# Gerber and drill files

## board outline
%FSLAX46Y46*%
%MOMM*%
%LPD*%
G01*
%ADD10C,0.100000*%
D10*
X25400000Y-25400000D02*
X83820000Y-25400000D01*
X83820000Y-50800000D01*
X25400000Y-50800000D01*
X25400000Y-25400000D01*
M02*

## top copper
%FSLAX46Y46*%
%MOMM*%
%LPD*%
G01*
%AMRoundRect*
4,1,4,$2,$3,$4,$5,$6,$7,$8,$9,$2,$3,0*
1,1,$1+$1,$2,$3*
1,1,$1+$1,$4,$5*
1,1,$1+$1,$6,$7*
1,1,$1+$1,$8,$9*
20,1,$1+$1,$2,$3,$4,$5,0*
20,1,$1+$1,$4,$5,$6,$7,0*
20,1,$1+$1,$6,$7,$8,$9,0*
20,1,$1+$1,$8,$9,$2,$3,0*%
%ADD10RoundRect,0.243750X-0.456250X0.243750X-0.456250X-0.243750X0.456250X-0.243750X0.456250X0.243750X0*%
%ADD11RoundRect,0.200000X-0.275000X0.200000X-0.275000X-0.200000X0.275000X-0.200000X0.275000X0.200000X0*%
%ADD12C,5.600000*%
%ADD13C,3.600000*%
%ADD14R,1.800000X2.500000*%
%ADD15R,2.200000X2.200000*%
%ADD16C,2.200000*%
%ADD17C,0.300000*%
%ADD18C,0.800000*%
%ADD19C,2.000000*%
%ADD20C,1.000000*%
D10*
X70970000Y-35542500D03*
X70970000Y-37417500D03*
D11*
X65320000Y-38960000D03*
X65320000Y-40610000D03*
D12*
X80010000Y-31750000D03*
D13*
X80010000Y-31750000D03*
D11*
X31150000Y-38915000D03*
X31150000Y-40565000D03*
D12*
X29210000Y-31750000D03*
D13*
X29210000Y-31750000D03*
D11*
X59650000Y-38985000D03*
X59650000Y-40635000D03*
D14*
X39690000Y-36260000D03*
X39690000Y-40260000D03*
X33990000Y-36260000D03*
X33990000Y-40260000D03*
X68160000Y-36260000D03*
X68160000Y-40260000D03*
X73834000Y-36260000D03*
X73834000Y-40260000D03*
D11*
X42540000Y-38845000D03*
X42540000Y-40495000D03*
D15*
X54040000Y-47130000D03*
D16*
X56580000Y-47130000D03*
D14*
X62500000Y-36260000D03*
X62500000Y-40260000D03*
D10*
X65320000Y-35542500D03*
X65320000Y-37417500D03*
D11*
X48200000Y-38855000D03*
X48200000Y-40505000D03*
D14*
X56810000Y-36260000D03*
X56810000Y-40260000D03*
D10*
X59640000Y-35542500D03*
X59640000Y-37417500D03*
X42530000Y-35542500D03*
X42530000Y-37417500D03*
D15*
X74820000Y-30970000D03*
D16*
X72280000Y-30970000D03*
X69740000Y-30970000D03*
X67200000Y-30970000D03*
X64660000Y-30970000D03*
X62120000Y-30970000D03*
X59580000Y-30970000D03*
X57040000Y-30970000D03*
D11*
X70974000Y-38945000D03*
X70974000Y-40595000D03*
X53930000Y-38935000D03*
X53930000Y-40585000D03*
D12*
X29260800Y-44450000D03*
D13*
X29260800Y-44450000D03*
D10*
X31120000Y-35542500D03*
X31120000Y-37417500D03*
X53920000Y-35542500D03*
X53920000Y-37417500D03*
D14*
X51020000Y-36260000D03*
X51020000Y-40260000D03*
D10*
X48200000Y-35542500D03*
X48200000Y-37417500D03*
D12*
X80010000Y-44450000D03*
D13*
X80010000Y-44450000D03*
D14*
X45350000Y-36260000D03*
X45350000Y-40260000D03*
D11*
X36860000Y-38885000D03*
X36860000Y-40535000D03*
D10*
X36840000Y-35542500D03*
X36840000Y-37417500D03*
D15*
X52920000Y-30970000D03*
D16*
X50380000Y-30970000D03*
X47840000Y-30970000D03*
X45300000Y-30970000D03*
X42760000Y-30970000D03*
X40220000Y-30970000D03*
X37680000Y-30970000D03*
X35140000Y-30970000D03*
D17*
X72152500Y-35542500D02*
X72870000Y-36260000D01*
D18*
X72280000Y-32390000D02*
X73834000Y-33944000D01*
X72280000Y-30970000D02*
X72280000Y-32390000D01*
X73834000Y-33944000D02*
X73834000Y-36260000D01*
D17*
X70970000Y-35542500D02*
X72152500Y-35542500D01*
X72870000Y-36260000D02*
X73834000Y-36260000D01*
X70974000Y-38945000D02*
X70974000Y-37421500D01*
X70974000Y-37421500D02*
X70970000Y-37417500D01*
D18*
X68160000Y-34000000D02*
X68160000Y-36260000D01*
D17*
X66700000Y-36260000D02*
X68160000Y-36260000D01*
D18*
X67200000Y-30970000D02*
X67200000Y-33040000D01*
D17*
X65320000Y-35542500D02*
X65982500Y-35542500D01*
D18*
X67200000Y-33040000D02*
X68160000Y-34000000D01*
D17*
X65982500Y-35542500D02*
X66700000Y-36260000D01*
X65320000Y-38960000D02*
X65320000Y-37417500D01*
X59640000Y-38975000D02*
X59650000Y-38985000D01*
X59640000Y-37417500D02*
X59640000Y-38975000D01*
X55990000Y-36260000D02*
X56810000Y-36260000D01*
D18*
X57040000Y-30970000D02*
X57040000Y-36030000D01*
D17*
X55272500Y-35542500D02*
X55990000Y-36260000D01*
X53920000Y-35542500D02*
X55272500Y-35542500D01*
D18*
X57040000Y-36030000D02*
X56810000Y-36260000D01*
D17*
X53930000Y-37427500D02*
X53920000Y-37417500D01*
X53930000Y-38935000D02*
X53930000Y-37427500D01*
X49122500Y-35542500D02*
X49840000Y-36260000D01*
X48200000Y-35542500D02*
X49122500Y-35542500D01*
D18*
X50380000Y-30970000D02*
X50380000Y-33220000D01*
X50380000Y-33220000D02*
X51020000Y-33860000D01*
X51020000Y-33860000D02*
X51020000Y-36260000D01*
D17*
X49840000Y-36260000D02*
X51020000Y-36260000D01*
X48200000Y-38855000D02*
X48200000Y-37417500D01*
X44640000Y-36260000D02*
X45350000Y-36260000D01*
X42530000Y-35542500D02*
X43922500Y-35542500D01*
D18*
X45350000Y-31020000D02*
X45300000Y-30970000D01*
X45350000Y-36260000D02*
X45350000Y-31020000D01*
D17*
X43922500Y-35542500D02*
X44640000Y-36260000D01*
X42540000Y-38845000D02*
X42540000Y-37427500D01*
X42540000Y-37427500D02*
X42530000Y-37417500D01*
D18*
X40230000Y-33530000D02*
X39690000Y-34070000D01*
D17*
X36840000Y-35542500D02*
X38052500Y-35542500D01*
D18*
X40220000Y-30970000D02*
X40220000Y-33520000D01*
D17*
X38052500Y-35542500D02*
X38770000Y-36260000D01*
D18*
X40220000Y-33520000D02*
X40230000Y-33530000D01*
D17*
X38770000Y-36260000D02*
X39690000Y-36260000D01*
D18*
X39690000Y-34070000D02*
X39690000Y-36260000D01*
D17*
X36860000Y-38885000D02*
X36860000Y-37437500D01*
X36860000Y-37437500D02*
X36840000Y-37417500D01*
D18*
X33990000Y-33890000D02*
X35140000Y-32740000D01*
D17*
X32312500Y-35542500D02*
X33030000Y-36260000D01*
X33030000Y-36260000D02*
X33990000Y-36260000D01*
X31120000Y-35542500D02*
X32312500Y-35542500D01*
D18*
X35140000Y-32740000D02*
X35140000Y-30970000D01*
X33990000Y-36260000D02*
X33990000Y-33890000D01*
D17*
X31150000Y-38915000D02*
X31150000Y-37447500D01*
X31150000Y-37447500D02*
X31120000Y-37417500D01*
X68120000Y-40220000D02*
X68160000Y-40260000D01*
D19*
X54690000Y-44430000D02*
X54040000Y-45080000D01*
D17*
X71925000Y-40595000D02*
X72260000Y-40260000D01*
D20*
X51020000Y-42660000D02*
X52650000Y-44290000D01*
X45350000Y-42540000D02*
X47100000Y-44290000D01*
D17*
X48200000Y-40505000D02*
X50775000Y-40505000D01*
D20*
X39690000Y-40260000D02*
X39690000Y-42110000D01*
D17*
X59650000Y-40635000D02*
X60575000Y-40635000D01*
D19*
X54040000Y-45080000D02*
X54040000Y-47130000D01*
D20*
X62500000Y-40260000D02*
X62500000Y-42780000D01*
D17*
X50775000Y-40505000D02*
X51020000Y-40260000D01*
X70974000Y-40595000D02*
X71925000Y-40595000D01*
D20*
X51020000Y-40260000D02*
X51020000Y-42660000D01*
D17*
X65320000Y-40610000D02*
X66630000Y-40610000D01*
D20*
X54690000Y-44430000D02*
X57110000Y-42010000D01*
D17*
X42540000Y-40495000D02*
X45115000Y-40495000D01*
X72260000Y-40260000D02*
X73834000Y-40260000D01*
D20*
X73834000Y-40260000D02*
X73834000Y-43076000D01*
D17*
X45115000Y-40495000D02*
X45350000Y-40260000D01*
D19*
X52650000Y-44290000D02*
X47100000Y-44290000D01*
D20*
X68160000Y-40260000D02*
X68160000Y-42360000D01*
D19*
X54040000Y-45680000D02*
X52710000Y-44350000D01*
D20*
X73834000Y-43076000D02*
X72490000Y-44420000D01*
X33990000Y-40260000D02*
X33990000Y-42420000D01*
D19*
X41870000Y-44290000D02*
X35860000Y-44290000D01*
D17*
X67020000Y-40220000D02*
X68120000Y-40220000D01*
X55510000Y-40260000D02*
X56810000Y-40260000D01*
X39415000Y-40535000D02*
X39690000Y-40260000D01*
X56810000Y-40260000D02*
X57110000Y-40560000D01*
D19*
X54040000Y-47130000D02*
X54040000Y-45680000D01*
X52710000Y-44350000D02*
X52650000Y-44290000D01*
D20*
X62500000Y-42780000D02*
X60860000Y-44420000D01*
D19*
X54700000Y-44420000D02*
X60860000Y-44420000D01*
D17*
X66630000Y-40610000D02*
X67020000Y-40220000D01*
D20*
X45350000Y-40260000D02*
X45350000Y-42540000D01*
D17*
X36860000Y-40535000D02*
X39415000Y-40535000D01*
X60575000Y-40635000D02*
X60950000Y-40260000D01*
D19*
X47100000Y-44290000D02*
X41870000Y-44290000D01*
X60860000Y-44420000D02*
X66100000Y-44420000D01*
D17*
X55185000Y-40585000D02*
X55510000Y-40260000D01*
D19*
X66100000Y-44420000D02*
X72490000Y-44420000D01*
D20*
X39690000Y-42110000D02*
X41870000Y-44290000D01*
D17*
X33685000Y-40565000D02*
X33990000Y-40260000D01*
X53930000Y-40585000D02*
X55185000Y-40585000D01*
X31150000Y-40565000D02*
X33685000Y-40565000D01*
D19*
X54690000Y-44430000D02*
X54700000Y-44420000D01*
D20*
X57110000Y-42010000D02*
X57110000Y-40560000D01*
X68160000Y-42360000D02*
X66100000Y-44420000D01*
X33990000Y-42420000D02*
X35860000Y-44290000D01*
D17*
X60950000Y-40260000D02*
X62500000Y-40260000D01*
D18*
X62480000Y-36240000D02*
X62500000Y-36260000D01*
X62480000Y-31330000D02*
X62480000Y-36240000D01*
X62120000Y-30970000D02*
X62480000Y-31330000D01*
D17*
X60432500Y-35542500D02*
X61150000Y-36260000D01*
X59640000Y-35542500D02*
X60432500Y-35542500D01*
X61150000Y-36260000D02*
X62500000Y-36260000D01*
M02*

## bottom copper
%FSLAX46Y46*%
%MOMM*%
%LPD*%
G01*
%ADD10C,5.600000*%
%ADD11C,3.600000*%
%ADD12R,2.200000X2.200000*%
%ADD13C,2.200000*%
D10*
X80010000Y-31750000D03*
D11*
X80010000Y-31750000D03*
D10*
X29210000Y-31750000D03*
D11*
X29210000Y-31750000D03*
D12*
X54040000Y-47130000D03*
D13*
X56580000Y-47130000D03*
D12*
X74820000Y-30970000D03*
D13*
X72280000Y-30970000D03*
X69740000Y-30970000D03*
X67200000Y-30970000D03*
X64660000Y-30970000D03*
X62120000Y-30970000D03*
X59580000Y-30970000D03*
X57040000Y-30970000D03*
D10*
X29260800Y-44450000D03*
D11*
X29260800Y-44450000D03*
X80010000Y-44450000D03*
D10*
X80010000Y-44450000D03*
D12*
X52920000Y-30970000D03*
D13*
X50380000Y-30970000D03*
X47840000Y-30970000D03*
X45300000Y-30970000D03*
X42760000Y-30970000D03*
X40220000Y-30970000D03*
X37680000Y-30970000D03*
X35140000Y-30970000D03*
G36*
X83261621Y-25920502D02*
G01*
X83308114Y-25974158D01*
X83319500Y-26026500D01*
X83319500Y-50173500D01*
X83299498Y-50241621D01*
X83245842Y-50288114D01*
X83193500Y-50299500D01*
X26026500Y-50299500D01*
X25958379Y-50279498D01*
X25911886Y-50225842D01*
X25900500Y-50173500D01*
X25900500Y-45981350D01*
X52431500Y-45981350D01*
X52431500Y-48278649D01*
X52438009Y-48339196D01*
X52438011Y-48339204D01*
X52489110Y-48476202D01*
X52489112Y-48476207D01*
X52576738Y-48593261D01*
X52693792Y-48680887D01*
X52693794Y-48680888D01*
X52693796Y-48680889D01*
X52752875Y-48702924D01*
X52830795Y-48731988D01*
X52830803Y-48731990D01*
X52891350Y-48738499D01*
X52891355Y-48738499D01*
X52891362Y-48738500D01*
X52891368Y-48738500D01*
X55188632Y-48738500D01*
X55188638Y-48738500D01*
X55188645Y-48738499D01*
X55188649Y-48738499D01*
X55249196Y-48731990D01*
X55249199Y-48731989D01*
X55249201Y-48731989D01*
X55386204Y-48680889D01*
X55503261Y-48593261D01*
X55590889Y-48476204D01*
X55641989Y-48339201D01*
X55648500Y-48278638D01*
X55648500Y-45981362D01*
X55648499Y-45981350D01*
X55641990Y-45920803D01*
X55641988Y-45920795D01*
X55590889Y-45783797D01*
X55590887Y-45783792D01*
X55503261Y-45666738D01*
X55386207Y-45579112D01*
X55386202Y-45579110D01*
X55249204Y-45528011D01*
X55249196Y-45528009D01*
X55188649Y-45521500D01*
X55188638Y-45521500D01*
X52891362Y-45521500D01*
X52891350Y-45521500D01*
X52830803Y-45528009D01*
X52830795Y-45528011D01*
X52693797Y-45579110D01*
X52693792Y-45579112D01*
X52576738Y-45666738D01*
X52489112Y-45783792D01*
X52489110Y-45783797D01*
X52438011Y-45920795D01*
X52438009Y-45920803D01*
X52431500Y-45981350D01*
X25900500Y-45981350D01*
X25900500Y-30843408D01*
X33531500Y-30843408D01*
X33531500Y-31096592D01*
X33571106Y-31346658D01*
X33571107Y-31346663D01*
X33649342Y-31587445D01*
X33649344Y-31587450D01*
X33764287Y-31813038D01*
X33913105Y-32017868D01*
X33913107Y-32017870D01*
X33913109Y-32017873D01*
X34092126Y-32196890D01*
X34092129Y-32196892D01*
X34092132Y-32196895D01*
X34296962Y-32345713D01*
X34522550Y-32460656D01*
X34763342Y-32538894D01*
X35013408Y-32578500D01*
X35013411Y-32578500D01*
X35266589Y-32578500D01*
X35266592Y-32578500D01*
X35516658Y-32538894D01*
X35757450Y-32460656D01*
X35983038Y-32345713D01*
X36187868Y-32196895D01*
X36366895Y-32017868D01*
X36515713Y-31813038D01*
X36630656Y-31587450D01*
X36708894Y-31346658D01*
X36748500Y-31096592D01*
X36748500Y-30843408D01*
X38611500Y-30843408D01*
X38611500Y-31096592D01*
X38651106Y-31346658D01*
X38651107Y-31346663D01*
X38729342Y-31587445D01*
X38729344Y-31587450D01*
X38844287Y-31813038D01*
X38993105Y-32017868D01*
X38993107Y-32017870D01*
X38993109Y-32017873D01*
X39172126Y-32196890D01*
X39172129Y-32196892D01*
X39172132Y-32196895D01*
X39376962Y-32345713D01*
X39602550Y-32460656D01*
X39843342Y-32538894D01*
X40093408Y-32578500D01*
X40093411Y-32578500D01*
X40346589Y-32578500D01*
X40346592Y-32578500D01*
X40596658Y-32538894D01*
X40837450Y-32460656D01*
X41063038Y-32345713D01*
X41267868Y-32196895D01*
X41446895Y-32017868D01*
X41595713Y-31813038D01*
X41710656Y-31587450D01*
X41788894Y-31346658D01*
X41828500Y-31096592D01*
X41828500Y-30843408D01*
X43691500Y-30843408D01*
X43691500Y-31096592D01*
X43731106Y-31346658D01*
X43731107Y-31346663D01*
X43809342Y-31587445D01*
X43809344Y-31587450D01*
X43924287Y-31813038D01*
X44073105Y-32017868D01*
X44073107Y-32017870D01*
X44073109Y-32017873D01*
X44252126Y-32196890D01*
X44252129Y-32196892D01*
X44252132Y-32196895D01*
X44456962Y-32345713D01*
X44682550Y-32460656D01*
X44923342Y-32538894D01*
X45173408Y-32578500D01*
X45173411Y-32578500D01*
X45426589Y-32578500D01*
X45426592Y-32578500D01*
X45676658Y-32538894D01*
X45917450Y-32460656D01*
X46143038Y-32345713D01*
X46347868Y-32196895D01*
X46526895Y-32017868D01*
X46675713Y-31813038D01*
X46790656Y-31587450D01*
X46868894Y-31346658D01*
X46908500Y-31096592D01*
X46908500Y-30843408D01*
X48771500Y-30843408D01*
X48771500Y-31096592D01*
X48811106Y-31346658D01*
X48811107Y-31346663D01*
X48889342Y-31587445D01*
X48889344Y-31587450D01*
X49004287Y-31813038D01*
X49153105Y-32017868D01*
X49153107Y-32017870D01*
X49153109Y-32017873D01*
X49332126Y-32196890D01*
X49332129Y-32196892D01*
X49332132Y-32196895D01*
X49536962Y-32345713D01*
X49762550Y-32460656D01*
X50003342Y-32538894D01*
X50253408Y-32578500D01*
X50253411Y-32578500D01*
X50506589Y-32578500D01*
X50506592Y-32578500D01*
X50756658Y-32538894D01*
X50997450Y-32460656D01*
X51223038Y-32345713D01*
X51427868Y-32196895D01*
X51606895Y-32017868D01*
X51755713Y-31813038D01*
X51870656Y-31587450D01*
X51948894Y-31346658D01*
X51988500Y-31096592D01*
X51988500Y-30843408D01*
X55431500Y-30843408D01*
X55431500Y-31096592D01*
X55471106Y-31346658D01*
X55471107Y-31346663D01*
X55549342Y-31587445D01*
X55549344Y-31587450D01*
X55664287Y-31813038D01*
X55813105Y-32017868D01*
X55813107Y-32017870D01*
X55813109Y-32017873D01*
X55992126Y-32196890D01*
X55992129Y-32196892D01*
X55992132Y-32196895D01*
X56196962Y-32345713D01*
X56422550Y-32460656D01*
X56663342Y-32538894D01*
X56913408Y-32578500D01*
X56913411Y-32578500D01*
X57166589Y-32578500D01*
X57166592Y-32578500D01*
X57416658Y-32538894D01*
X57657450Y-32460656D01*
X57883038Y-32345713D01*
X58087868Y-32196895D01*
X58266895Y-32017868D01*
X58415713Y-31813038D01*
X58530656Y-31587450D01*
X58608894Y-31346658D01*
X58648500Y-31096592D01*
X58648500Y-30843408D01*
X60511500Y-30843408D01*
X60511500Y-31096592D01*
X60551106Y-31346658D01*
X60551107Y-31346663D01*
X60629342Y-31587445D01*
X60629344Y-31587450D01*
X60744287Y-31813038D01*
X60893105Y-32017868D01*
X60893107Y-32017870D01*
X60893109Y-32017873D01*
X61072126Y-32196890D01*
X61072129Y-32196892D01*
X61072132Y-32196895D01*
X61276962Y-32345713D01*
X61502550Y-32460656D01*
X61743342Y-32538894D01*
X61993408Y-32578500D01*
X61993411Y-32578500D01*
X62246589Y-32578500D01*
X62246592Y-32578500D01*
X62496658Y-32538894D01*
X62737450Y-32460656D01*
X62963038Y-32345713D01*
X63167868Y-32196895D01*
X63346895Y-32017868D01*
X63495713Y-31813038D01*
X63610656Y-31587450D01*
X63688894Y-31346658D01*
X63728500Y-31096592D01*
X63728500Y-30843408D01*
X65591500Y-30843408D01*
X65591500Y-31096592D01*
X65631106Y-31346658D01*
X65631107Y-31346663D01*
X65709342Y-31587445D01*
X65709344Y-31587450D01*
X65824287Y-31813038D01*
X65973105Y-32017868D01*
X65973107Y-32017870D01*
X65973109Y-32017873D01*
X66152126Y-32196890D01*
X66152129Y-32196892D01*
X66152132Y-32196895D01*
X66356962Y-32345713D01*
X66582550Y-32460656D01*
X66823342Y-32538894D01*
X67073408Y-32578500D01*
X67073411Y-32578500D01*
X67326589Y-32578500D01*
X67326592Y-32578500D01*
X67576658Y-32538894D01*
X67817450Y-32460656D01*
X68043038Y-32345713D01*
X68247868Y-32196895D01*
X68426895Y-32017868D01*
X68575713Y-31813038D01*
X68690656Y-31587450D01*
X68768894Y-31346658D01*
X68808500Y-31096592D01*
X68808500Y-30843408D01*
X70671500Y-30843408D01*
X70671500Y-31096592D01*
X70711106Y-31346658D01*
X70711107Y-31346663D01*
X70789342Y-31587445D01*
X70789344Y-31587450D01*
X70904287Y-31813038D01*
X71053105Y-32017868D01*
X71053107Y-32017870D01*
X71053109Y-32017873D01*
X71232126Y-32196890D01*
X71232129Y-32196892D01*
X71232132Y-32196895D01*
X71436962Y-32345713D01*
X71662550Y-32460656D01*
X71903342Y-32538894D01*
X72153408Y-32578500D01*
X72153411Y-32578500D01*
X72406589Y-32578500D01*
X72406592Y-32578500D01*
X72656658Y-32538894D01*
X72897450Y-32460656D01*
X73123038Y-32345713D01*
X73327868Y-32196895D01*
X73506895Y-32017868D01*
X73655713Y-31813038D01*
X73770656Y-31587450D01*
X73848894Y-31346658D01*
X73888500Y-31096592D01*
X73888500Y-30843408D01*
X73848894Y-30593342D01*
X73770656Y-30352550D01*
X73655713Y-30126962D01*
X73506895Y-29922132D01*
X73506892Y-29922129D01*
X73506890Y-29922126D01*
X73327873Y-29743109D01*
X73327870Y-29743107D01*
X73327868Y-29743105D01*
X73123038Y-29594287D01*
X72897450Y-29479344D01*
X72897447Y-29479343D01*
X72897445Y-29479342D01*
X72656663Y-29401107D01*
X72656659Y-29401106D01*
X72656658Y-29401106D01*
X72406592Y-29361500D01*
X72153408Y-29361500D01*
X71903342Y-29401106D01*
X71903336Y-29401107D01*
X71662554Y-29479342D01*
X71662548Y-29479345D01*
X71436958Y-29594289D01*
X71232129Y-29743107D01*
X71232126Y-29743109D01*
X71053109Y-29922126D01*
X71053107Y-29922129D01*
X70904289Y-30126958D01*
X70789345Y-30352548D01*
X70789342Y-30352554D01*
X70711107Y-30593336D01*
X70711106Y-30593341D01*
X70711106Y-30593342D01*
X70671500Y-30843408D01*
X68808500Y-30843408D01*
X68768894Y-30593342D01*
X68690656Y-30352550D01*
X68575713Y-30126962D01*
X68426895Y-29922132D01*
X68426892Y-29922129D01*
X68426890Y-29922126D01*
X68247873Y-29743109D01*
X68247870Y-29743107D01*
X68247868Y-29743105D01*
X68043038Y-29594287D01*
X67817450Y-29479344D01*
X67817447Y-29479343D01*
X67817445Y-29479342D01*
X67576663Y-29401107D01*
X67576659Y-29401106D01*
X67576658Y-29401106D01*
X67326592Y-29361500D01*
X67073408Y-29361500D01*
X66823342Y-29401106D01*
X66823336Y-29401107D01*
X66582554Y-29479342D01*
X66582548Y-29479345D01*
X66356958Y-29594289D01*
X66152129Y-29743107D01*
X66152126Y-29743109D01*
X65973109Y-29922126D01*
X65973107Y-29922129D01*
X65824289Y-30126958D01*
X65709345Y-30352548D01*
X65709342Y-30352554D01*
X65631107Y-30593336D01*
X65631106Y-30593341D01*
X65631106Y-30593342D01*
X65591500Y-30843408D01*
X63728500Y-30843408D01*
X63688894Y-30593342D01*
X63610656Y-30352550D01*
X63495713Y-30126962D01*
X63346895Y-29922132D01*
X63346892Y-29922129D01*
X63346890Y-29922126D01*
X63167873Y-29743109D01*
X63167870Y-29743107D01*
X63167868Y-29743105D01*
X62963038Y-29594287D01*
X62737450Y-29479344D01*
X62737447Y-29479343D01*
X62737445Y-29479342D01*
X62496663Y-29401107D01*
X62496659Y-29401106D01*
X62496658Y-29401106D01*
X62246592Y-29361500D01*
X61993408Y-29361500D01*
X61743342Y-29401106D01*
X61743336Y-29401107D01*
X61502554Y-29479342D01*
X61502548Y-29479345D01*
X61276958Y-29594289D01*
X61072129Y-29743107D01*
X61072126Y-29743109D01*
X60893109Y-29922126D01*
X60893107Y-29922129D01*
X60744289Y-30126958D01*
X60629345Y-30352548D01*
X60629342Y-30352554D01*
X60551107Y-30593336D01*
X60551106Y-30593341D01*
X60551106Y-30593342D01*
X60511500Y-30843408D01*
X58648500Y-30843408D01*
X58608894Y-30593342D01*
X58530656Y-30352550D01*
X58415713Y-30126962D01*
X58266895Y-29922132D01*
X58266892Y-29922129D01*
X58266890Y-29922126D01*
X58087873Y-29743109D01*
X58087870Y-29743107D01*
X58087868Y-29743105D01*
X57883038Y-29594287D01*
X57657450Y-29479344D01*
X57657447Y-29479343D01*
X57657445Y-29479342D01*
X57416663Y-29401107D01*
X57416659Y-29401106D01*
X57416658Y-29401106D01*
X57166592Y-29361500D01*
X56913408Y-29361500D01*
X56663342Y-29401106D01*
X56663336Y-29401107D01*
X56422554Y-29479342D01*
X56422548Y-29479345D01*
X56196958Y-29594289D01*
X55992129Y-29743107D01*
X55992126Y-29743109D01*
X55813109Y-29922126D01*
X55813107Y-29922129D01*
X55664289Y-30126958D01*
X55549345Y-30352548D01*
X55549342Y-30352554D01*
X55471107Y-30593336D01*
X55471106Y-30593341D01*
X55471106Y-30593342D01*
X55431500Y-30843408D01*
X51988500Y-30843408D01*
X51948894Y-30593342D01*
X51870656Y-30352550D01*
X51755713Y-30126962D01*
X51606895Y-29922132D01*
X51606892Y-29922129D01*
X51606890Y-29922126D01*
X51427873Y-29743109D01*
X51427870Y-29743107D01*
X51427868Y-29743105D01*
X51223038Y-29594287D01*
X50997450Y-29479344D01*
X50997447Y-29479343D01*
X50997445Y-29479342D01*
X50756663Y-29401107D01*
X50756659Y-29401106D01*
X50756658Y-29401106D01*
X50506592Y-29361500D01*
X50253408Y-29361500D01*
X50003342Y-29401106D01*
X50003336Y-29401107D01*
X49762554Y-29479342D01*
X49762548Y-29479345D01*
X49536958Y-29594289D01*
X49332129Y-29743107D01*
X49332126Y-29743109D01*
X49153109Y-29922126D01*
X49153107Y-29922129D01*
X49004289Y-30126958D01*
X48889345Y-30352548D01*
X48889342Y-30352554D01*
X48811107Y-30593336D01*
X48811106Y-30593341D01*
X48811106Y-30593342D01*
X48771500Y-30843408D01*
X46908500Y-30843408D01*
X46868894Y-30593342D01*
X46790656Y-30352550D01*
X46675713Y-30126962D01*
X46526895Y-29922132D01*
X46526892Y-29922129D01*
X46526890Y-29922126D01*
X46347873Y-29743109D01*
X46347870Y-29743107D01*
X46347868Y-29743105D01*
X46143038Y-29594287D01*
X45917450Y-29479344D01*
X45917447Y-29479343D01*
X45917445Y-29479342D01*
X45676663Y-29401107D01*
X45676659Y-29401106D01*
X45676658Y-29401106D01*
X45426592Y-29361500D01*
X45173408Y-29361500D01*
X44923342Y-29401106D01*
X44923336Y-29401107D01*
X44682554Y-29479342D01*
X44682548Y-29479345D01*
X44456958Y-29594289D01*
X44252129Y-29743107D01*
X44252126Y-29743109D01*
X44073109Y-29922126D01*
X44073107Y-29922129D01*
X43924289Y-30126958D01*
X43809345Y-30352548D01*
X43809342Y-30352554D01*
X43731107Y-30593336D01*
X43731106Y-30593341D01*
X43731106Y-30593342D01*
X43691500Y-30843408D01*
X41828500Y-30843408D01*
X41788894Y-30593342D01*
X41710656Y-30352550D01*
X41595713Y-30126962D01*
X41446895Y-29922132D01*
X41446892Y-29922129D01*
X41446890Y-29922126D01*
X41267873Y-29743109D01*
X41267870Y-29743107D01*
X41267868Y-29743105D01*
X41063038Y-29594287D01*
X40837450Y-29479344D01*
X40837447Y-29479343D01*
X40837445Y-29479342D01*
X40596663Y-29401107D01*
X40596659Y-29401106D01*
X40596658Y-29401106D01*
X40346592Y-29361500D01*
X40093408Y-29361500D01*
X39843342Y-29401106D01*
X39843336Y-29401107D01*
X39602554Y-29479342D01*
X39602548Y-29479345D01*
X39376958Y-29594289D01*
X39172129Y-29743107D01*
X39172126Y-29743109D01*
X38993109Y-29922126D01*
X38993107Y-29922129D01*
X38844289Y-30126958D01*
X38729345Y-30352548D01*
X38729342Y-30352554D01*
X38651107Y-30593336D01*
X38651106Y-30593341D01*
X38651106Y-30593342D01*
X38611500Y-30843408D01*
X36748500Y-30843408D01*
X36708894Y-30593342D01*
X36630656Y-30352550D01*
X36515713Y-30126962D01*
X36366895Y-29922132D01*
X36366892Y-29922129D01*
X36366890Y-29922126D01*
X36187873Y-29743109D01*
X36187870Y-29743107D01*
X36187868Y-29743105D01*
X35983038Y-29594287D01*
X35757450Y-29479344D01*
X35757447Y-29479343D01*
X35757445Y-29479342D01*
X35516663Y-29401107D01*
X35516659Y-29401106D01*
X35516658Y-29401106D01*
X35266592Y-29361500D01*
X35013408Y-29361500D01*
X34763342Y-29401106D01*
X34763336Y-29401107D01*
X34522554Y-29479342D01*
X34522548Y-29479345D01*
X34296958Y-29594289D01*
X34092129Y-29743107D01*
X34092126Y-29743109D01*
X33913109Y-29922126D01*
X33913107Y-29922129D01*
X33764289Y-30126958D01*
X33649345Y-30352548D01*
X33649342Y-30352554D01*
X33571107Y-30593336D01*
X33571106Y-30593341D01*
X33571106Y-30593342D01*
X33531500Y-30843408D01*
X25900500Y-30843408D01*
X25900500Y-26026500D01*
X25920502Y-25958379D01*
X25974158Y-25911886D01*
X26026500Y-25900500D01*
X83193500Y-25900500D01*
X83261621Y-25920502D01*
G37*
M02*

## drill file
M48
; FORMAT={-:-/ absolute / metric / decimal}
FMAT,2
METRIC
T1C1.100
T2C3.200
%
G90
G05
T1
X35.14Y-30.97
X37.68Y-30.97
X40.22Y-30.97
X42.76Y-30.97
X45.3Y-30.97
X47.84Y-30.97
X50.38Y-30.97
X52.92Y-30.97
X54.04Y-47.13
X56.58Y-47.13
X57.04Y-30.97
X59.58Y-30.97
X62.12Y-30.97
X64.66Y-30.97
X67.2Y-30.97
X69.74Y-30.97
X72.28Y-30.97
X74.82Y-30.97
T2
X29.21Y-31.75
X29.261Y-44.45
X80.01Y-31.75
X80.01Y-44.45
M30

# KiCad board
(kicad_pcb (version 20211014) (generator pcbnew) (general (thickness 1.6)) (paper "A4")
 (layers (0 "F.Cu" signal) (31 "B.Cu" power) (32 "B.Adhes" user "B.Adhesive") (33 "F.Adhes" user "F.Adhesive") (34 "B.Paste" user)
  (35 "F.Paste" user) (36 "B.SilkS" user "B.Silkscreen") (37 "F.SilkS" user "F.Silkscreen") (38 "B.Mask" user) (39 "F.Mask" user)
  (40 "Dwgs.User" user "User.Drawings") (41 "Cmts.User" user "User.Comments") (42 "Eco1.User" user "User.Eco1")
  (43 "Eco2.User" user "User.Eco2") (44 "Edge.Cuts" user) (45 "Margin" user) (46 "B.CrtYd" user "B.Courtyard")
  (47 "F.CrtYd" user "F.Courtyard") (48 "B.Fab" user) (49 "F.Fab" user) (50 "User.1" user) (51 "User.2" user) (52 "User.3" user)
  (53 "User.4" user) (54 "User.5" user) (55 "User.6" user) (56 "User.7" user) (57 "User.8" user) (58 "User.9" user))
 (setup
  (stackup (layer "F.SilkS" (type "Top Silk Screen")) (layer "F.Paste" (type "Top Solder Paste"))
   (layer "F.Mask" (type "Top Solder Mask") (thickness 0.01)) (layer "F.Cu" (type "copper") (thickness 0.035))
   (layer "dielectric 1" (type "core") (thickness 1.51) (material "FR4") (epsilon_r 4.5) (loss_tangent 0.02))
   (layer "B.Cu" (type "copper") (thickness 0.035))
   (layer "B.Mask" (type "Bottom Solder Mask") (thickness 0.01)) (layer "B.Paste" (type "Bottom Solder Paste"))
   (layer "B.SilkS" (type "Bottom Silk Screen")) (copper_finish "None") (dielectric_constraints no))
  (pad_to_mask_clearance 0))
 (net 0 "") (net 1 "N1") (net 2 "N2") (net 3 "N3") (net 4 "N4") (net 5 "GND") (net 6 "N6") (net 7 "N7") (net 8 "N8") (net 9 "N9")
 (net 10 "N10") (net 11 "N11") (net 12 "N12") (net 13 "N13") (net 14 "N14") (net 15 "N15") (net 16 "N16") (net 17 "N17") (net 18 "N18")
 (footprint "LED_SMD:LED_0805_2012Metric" (layer "F.Cu") (at 70.97 36.48 -90)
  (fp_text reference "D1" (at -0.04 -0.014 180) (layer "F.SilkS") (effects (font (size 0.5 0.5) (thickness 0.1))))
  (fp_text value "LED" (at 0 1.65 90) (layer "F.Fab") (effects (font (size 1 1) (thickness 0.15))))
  (pad "1" smd roundrect (at -0.9375 0 270) (size 0.975 1.4) (layers "F.Cu" "F.Paste" "F.Mask") (roundrect_rratio 0.25) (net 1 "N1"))
  (pad "2" smd roundrect (at 0.9375 0 270) (size 0.975 1.4) (layers "F.Cu" "F.Paste" "F.Mask") (roundrect_rratio 0.25) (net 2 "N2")))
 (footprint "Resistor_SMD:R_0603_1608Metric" (layer "F.Cu") (at 65.32 39.785 -90)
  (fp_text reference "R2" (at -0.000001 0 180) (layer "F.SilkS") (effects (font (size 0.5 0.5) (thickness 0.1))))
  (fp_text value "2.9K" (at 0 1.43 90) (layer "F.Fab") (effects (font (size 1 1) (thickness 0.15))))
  (pad "1" smd roundrect (at -0.825 0 270) (size 0.8 0.95) (layers "F.Cu" "F.Paste" "F.Mask") (roundrect_rratio 0.25) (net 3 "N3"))
  (pad "2" smd roundrect (at 0.825 0 270) (size 0.8 0.95) (layers "F.Cu" "F.Paste" "F.Mask") (roundrect_rratio 0.25) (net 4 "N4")))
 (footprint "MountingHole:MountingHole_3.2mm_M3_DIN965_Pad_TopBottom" (layer "F.Cu") (at 80.01 31.75)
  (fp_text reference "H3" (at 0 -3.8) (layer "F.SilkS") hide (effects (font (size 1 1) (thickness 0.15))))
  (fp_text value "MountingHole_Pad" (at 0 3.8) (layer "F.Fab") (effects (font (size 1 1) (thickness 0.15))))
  (pad "1" connect circle (at 0 0) (size 5.6 5.6) (layers "B.Cu" "B.Mask") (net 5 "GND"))
  (pad "1" connect circle (at 0 0) (size 5.6 5.6) (layers "F.Cu" "F.Mask") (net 5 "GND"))
  (pad "1" thru_hole circle (at 0 0) (size 3.6 3.6) (drill 3.2) (layers *.Cu *.Mask) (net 5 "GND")))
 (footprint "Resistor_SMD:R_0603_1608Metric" (layer "F.Cu") (at 31.15 39.74 -90)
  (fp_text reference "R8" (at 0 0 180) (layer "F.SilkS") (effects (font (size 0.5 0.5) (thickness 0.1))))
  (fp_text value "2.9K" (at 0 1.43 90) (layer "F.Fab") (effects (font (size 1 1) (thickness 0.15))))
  (pad "1" smd roundrect (at -0.825 0 270) (size 0.8 0.95) (layers "F.Cu" "F.Paste" "F.Mask") (roundrect_rratio 0.25) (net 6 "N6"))
  (pad "2" smd roundrect (at 0.825 0 270) (size 0.8 0.95) (layers "F.Cu" "F.Paste" "F.Mask") (roundrect_rratio 0.25) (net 4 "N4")))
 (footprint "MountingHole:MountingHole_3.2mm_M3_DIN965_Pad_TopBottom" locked (layer "F.Cu") (at 29.21 31.75)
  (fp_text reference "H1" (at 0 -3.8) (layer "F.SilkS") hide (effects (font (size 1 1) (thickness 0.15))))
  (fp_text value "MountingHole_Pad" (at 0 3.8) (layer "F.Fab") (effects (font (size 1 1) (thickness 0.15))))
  (pad "1" connect circle locked (at 0 0) (size 5.6 5.6) (layers "F.Cu" "F.Mask") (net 5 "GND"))
  (pad "1" connect circle locked (at 0 0) (size 5.6 5.6) (layers "B.Cu" "B.Mask") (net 5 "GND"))
  (pad "1" thru_hole circle locked (at 0 0) (size 3.6 3.6) (drill 3.2) (layers *.Cu *.Mask) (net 5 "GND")))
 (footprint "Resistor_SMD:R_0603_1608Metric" (layer "F.Cu") (at 59.65 39.81 -90)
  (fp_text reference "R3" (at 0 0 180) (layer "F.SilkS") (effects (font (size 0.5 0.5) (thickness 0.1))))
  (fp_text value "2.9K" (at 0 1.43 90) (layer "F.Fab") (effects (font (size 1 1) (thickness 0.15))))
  (pad "1" smd roundrect (at -0.825 0 270) (size 0.8 0.95) (layers "F.Cu" "F.Paste" "F.Mask") (roundrect_rratio 0.25) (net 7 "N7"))
  (pad "2" smd roundrect (at 0.825 0 270) (size 0.8 0.95) (layers "F.Cu" "F.Paste" "F.Mask") (roundrect_rratio 0.25) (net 4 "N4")))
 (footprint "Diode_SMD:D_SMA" (layer "F.Cu") (at 39.69 38.26 -90)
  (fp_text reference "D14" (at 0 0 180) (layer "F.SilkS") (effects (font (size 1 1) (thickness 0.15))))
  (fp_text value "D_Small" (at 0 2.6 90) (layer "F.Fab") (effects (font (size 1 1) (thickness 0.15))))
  (pad "1" smd rect (at -2 0 270) (size 2.5 1.8) (layers "F.Cu" "F.Paste" "F.Mask") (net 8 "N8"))
  (pad "2" smd rect (at 2 0 270) (size 2.5 1.8) (layers "F.Cu" "F.Paste" "F.Mask") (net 4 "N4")))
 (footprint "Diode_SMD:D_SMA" (layer "F.Cu") (at 33.99 38.26 -90)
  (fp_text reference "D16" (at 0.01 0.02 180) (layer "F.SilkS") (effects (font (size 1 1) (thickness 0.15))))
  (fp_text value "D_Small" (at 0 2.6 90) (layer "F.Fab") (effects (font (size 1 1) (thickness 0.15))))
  (pad "1" smd rect (at -2 0 270) (size 2.5 1.8) (layers "F.Cu" "F.Paste" "F.Mask") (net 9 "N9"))
  (pad "2" smd rect (at 2 0 270) (size 2.5 1.8) (layers "F.Cu" "F.Paste" "F.Mask") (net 4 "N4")))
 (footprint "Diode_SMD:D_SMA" (layer "F.Cu") (at 68.16 38.26 -90)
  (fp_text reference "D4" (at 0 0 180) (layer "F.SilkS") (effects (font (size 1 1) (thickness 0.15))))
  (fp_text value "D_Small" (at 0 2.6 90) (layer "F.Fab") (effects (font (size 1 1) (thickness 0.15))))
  (pad "1" smd rect (at -2 0 270) (size 2.5 1.8) (layers "F.Cu" "F.Paste" "F.Mask") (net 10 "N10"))
  (pad "2" smd rect (at 2 0 270) (size 2.5 1.8) (layers "F.Cu" "F.Paste" "F.Mask") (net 4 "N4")))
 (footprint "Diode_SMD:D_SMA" (layer "F.Cu") (at 73.834 38.26 -90)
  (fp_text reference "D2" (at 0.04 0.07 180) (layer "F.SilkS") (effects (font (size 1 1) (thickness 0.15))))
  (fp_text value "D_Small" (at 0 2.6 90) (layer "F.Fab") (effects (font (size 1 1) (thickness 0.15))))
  (pad "1" smd rect (at -2 0 270) (size 2.5 1.8) (layers "F.Cu" "F.Paste" "F.Mask") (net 1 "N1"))
  (pad "2" smd rect (at 2 0 270) (size 2.5 1.8) (layers "F.Cu" "F.Paste" "F.Mask") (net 4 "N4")))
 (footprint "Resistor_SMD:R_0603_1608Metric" (layer "F.Cu") (at 42.54 39.67 -90)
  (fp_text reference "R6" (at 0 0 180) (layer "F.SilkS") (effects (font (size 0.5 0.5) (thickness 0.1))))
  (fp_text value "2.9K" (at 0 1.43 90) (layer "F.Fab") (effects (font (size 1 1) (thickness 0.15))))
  (pad "1" smd roundrect (at -0.825 0 270) (size 0.8 0.95) (layers "F.Cu" "F.Paste" "F.Mask") (roundrect_rratio 0.25) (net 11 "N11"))
  (pad "2" smd roundrect (at 0.825 0 270) (size 0.8 0.95) (layers "F.Cu" "F.Paste" "F.Mask") (roundrect_rratio 0.25) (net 4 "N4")))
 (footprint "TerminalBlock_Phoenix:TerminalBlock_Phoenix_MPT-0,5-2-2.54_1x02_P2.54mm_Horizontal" (layer "F.Cu") (at 54.04 47.13)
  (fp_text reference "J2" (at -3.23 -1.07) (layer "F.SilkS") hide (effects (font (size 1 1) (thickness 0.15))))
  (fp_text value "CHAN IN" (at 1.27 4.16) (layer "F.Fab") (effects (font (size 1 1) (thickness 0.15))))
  (pad "1" thru_hole rect (at 0 0) (size 2.2 2.2) (drill 1.1) (layers *.Cu *.Mask) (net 4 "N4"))
  (pad "2" thru_hole circle (at 2.54 0) (size 2.2 2.2) (drill 1.1) (layers *.Cu *.Mask) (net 5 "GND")))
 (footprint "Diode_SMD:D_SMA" (layer "F.Cu") (at 62.5 38.26 -90)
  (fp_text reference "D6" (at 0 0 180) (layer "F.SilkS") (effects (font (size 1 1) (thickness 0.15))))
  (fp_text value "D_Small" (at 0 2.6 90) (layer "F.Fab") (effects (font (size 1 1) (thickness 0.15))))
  (pad "1" smd rect (at -2 0 270) (size 2.5 1.8) (layers "F.Cu" "F.Paste" "F.Mask") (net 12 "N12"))
  (pad "2" smd rect (at 2 0 270) (size 2.5 1.8) (layers "F.Cu" "F.Paste" "F.Mask") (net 4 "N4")))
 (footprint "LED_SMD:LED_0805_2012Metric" (layer "F.Cu") (at 65.32 36.48 -90)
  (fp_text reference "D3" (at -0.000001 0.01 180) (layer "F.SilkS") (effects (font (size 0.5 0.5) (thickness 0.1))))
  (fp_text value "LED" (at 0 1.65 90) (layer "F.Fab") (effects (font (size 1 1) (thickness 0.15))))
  (pad "1" smd roundrect (at -0.9375 0 270) (size 0.975 1.4) (layers "F.Cu" "F.Paste" "F.Mask") (roundrect_rratio 0.25) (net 10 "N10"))
  (pad "2" smd roundrect (at 0.9375 0 270) (size 0.975 1.4) (layers "F.Cu" "F.Paste" "F.Mask") (roundrect_rratio 0.25) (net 3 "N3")))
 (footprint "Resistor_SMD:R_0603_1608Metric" (layer "F.Cu") (at 48.2 39.68 -90)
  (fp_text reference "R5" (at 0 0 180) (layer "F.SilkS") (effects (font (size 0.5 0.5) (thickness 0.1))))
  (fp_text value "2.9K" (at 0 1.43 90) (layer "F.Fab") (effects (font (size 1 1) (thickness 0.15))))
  (pad "1" smd roundrect (at -0.825 0 270) (size 0.8 0.95) (layers "F.Cu" "F.Paste" "F.Mask") (roundrect_rratio 0.25) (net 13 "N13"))
  (pad "2" smd roundrect (at 0.825 0 270) (size 0.8 0.95) (layers "F.Cu" "F.Paste" "F.Mask") (roundrect_rratio 0.25) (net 4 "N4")))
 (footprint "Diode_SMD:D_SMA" (layer "F.Cu") (at 56.81 38.26 -90)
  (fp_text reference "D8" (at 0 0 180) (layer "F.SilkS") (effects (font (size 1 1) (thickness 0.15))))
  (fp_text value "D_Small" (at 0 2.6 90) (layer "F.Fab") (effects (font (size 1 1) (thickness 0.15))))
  (pad "1" smd rect (at -2 0 270) (size 2.5 1.8) (layers "F.Cu" "F.Paste" "F.Mask") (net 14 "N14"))
  (pad "2" smd rect (at 2 0 270) (size 2.5 1.8) (layers "F.Cu" "F.Paste" "F.Mask") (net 4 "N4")))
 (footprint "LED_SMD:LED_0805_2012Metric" (layer "F.Cu") (at 59.64 36.48 -90)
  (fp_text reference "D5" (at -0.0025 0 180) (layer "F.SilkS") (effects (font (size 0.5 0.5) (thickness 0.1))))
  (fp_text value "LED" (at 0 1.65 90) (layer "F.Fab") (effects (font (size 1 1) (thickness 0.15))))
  (pad "1" smd roundrect (at -0.9375 0 270) (size 0.975 1.4) (layers "F.Cu" "F.Paste" "F.Mask") (roundrect_rratio 0.25) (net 12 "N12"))
  (pad "2" smd roundrect (at 0.9375 0 270) (size 0.975 1.4) (layers "F.Cu" "F.Paste" "F.Mask") (roundrect_rratio 0.25) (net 7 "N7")))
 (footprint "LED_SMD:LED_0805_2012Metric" (layer "F.Cu") (at 42.53 36.48 -90)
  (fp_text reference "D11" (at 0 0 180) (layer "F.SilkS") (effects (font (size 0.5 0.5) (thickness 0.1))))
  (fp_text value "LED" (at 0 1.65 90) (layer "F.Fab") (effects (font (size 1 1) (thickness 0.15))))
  (pad "1" smd roundrect (at -0.9375 0 270) (size 0.975 1.4) (layers "F.Cu" "F.Paste" "F.Mask") (roundrect_rratio 0.25) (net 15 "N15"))
  (pad "2" smd roundrect (at 0.9375 0 270) (size 0.975 1.4) (layers "F.Cu" "F.Paste" "F.Mask") (roundrect_rratio 0.25) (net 11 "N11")))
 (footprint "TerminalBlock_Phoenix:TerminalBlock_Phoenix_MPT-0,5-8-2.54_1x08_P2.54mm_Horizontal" (layer "F.Cu") (at 74.82 30.97 180)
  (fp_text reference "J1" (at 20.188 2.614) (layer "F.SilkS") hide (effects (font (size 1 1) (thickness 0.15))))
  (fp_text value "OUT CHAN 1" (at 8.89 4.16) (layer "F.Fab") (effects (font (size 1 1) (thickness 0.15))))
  (pad "1" thru_hole rect (at 0 0 180) (size 2.2 2.2) (drill 1.1) (layers *.Cu *.Mask) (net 5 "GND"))
  (pad "2" thru_hole circle (at 2.54 0 180) (size 2.2 2.2) (drill 1.1) (layers *.Cu *.Mask) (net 1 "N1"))
  (pad "3" thru_hole circle (at 5.08 0 180) (size 2.2 2.2) (drill 1.1) (layers *.Cu *.Mask) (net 5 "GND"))
  (pad "4" thru_hole circle (at 7.62 0 180) (size 2.2 2.2) (drill 1.1) (layers *.Cu *.Mask) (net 10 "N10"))
  (pad "5" thru_hole circle (at 10.16 0 180) (size 2.2 2.2) (drill 1.1) (layers *.Cu *.Mask) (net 5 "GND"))
  (pad "6" thru_hole circle (at 12.7 0 180) (size 2.2 2.2) (drill 1.1) (layers *.Cu *.Mask) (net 12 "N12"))
  (pad "7" thru_hole circle (at 15.24 0 180) (size 2.2 2.2) (drill 1.1) (layers *.Cu *.Mask) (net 5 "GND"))
  (pad "8" thru_hole circle (at 17.78 0 180) (size 2.2 2.2) (drill 1.1) (layers *.Cu *.Mask) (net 14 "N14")))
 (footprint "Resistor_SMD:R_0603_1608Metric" (layer "F.Cu") (at 70.974 39.77 -90)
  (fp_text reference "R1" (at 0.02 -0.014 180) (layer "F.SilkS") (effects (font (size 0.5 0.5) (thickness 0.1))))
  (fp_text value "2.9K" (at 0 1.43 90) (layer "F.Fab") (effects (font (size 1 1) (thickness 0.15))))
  (pad "1" smd roundrect (at -0.825 0 270) (size 0.8 0.95) (layers "F.Cu" "F.Paste" "F.Mask") (roundrect_rratio 0.25) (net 2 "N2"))
  (pad "2" smd roundrect (at 0.825 0 270) (size 0.8 0.95) (layers "F.Cu" "F.Paste" "F.Mask") (roundrect_rratio 0.25) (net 4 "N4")))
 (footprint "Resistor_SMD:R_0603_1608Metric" (layer "F.Cu") (at 53.93 39.76 -90)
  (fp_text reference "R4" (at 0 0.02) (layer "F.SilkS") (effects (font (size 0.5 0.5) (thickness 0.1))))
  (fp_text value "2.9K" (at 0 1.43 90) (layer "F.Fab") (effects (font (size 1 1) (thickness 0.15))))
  (pad "1" smd roundrect (at -0.825 0 270) (size 0.8 0.95) (layers "F.Cu" "F.Paste" "F.Mask") (roundrect_rratio 0.25) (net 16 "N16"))
  (pad "2" smd roundrect (at 0.825 0 270) (size 0.8 0.95) (layers "F.Cu" "F.Paste" "F.Mask") (roundrect_rratio 0.25) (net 4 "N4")))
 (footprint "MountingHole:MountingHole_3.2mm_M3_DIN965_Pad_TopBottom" (layer "F.Cu") (at 29.2608 44.45)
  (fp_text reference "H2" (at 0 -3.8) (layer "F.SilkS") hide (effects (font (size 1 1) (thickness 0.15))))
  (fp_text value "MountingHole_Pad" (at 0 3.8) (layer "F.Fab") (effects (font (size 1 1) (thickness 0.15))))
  (pad "1" connect circle (at 0 0) (size 5.6 5.6) (layers "F.Cu" "F.Mask") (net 5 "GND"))
  (pad "1" connect circle (at 0 0) (size 5.6 5.6) (layers "B.Cu" "B.Mask") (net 5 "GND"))
  (pad "1" thru_hole circle (at 0 0) (size 3.6 3.6) (drill 3.2) (layers *.Cu *.Mask) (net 5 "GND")))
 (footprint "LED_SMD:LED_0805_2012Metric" (layer "F.Cu") (at 31.12 36.48 -90)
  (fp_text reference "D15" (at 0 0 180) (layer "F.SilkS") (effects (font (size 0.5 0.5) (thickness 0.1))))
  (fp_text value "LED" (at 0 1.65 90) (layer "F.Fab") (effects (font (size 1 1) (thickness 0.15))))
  (pad "1" smd roundrect (at -0.9375 0 270) (size 0.975 1.4) (layers "F.Cu" "F.Paste" "F.Mask") (roundrect_rratio 0.25) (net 9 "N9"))
  (pad "2" smd roundrect (at 0.9375 0 270) (size 0.975 1.4) (layers "F.Cu" "F.Paste" "F.Mask") (roundrect_rratio 0.25) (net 6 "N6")))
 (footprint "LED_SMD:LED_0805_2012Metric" (layer "F.Cu") (at 53.92 36.48 -90)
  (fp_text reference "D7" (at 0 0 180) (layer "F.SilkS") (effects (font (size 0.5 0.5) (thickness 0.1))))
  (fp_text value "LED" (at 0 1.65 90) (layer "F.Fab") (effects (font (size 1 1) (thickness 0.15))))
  (pad "1" smd roundrect (at -0.9375 0 270) (size 0.975 1.4) (layers "F.Cu" "F.Paste" "F.Mask") (roundrect_rratio 0.25) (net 14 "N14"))
  (pad "2" smd roundrect (at 0.9375 0 270) (size 0.975 1.4) (layers "F.Cu" "F.Paste" "F.Mask") (roundrect_rratio 0.25) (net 16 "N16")))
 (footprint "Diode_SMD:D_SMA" (layer "F.Cu") (at 51.02 38.26 -90)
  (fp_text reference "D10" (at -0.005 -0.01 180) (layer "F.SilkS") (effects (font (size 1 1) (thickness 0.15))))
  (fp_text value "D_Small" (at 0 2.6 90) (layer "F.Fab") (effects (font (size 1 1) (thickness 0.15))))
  (pad "1" smd rect (at -2 0 270) (size 2.5 1.8) (layers "F.Cu" "F.Paste" "F.Mask") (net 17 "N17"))
  (pad "2" smd rect (at 2 0 270) (size 2.5 1.8) (layers "F.Cu" "F.Paste" "F.Mask") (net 4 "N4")))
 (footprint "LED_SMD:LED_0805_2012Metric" (layer "F.Cu") (at 48.2 36.48 -90)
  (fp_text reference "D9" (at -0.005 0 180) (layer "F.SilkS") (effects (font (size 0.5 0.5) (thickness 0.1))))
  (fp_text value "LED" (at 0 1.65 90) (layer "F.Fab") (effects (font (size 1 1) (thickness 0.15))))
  (pad "1" smd roundrect (at -0.9375 0 270) (size 0.975 1.4) (layers "F.Cu" "F.Paste" "F.Mask") (roundrect_rratio 0.25) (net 17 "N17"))
  (pad "2" smd roundrect (at 0.9375 0 270) (size 0.975 1.4) (layers "F.Cu" "F.Paste" "F.Mask") (roundrect_rratio 0.25) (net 13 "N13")))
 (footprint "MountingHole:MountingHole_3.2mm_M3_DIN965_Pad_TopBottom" (layer "F.Cu") (at 80.01 44.45)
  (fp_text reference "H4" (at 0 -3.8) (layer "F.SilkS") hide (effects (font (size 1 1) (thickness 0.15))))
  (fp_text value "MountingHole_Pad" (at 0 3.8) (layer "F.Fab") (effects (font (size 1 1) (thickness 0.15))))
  (pad "1" connect circle (at 0 0) (size 5.6 5.6) (layers "F.Cu" "F.Mask") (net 5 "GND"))
  (pad "1" thru_hole circle (at 0 0) (size 3.6 3.6) (drill 3.2) (layers *.Cu *.Mask) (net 5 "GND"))
  (pad "1" connect circle (at 0 0) (size 5.6 5.6) (layers "B.Cu" "B.Mask") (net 5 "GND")))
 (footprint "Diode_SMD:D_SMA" (layer "F.Cu") (at 45.35 38.26 -90)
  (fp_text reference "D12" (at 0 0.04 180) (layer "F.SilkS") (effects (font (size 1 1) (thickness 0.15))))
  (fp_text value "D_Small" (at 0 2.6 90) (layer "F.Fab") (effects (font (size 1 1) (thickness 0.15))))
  (pad "1" smd rect (at -2 0 270) (size 2.5 1.8) (layers "F.Cu" "F.Paste" "F.Mask") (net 15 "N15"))
  (pad "2" smd rect (at 2 0 270) (size 2.5 1.8) (layers "F.Cu" "F.Paste" "F.Mask") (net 4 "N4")))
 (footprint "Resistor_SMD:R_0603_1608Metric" (layer "F.Cu") (at 36.86 39.71 -90)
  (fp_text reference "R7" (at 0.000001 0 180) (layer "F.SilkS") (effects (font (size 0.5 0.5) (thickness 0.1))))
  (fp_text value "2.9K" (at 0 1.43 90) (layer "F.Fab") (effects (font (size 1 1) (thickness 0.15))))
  (pad "1" smd roundrect (at -0.825 0 270) (size 0.8 0.95) (layers "F.Cu" "F.Paste" "F.Mask") (roundrect_rratio 0.25) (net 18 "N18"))
  (pad "2" smd roundrect (at 0.825 0 270) (size 0.8 0.95) (layers "F.Cu" "F.Paste" "F.Mask") (roundrect_rratio 0.25) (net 4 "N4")))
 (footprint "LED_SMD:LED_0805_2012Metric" (layer "F.Cu") (at 36.84 36.48 -90)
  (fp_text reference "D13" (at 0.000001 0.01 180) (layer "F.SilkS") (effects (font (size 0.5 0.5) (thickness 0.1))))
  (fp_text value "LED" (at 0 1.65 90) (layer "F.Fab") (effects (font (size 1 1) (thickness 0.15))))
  (pad "1" smd roundrect (at -0.9375 0 270) (size 0.975 1.4) (layers "F.Cu" "F.Paste" "F.Mask") (roundrect_rratio 0.25) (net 8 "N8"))
  (pad "2" smd roundrect (at 0.9375 0 270) (size 0.975 1.4) (layers "F.Cu" "F.Paste" "F.Mask") (roundrect_rratio 0.25) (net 18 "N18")))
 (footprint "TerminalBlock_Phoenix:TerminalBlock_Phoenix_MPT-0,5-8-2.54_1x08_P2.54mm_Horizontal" (layer "F.Cu") (at 52.92 30.97 180)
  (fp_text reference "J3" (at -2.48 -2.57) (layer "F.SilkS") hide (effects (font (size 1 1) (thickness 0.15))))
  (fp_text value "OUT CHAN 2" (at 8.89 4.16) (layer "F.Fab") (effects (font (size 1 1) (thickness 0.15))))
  (pad "1" thru_hole rect (at 0 0 180) (size 2.2 2.2) (drill 1.1) (layers *.Cu *.Mask) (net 5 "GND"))
  (pad "2" thru_hole circle (at 2.54 0 180) (size 2.2 2.2) (drill 1.1) (layers *.Cu *.Mask) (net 17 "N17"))
  (pad "3" thru_hole circle (at 5.08 0 180) (size 2.2 2.2) (drill 1.1) (layers *.Cu *.Mask) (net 5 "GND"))
  (pad "4" thru_hole circle (at 7.62 0 180) (size 2.2 2.2) (drill 1.1) (layers *.Cu *.Mask) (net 15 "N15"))
  (pad "5" thru_hole circle (at 10.16 0 180) (size 2.2 2.2) (drill 1.1) (layers *.Cu *.Mask) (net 5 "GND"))
  (pad "6" thru_hole circle (at 12.7 0 180) (size 2.2 2.2) (drill 1.1) (layers *.Cu *.Mask) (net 8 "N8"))
  (pad "7" thru_hole circle (at 15.24 0 180) (size 2.2 2.2) (drill 1.1) (layers *.Cu *.Mask) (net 5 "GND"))
  (pad "8" thru_hole circle (at 17.78 0 180) (size 2.2 2.2) (drill 1.1) (layers *.Cu *.Mask) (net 9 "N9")))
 (gr_rect (start 25.4 25.4) (end 83.82 50.8) (layer "Edge.Cuts") (width 0.1) (fill none))
 (segment (start 72.1525 35.5425) (end 72.87 36.26) (width 0.3) (layer "F.Cu") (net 1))
 (segment (start 72.28 32.39) (end 73.834 33.944) (width 0.8) (layer "F.Cu") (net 1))
 (segment (start 72.28 30.97) (end 72.28 32.39) (width 0.8) (layer "F.Cu") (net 1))
 (segment (start 73.834 33.944) (end 73.834 36.26) (width 0.8) (layer "F.Cu") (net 1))
 (segment (start 70.97 35.5425) (end 72.1525 35.5425) (width 0.3) (layer "F.Cu") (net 1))
 (segment (start 72.87 36.26) (end 73.834 36.26) (width 0.3) (layer "F.Cu") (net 1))
 (segment (start 70.974 38.945) (end 70.974 37.4215) (width 0.3) (layer "F.Cu") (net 2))
 (segment (start 70.974 37.4215) (end 70.97 37.4175) (width 0.3) (layer "F.Cu") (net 2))
 (segment (start 68.16 34) (end 68.16 36.26) (width 0.8) (layer "F.Cu") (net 10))
 (segment (start 66.7 36.26) (end 68.16 36.26) (width 0.3) (layer "F.Cu") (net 10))
 (segment (start 67.2 30.97) (end 67.2 33.04) (width 0.8) (layer "F.Cu") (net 10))
 (segment (start 65.32 35.5425) (end 65.9825 35.5425) (width 0.3) (layer "F.Cu") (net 10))
 (segment (start 67.2 33.04) (end 68.16 34) (width 0.8) (layer "F.Cu") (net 10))
 (segment (start 65.9825 35.5425) (end 66.7 36.26) (width 0.3) (layer "F.Cu") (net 10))
 (segment (start 65.32 38.96) (end 65.32 37.4175) (width 0.3) (layer "F.Cu") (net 3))
 (segment (start 59.64 38.975) (end 59.65 38.985) (width 0.3) (layer "F.Cu") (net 7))
 (segment (start 59.64 37.4175) (end 59.64 38.975) (width 0.3) (layer "F.Cu") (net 7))
 (segment (start 55.99 36.26) (end 56.81 36.26) (width 0.3) (layer "F.Cu") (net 14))
 (segment (start 57.04 30.97) (end 57.04 36.03) (width 0.8) (layer "F.Cu") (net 14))
 (segment (start 55.2725 35.5425) (end 55.99 36.26) (width 0.3) (layer "F.Cu") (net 14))
 (segment (start 53.92 35.5425) (end 55.2725 35.5425) (width 0.3) (layer "F.Cu") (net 14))
 (segment (start 57.04 36.03) (end 56.81 36.26) (width 0.8) (layer "F.Cu") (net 14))
 (segment (start 53.93 37.4275) (end 53.92 37.4175) (width 0.3) (layer "F.Cu") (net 16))
 (segment (start 53.93 38.935) (end 53.93 37.4275) (width 0.3) (layer "F.Cu") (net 16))
 (segment (start 49.1225 35.5425) (end 49.84 36.26) (width 0.3) (layer "F.Cu") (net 17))
 (segment (start 48.2 35.5425) (end 49.1225 35.5425) (width 0.3) (layer "F.Cu") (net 17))
 (segment (start 50.38 30.97) (end 50.38 33.22) (width 0.8) (layer "F.Cu") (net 17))
 (segment (start 50.38 33.22) (end 51.02 33.86) (width 0.8) (layer "F.Cu") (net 17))
 (segment (start 51.02 33.86) (end 51.02 36.26) (width 0.8) (layer "F.Cu") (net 17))
 (segment (start 49.84 36.26) (end 51.02 36.26) (width 0.3) (layer "F.Cu") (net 17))
 (segment (start 48.2 38.855) (end 48.2 37.4175) (width 0.3) (layer "F.Cu") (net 13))
 (segment (start 44.64 36.26) (end 45.35 36.26) (width 0.3) (layer "F.Cu") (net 15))
 (segment (start 42.53 35.5425) (end 43.9225 35.5425) (width 0.3) (layer "F.Cu") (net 15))
 (segment (start 45.35 31.02) (end 45.3 30.97) (width 0.8) (layer "F.Cu") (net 15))
 (segment (start 45.35 36.26) (end 45.35 31.02) (width 0.8) (layer "F.Cu") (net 15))
 (segment (start 43.9225 35.5425) (end 44.64 36.26) (width 0.3) (layer "F.Cu") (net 15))
 (segment (start 42.54 38.845) (end 42.54 37.4275) (width 0.3) (layer "F.Cu") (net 11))
 (segment (start 42.54 37.4275) (end 42.53 37.4175) (width 0.3) (layer "F.Cu") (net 11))
 (segment (start 40.23 33.53) (end 39.69 34.07) (width 0.8) (layer "F.Cu") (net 8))
 (segment (start 36.84 35.5425) (end 38.0525 35.5425) (width 0.3) (layer "F.Cu") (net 8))
 (segment (start 40.22 30.97) (end 40.22 33.52) (width 0.8) (layer "F.Cu") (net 8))
 (segment (start 38.0525 35.5425) (end 38.77 36.26) (width 0.3) (layer "F.Cu") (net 8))
 (segment (start 40.22 33.52) (end 40.23 33.53) (width 0.8) (layer "F.Cu") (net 8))
 (segment (start 38.77 36.26) (end 39.69 36.26) (width 0.3) (layer "F.Cu") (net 8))
 (segment (start 39.69 34.07) (end 39.69 36.26) (width 0.8) (layer "F.Cu") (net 8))
 (segment (start 36.86 38.885) (end 36.86 37.4375) (width 0.3) (layer "F.Cu") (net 18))
 (segment (start 36.86 37.4375) (end 36.84 37.4175) (width 0.3) (layer "F.Cu") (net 18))
 (segment (start 33.99 33.89) (end 35.14 32.74) (width 0.8) (layer "F.Cu") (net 9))
 (segment (start 32.3125 35.5425) (end 33.03 36.26) (width 0.3) (layer "F.Cu") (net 9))
 (segment (start 33.03 36.26) (end 33.99 36.26) (width 0.3) (layer "F.Cu") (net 9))
 (segment (start 31.12 35.5425) (end 32.3125 35.5425) (width 0.3) (layer "F.Cu") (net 9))
 (segment (start 35.14 32.74) (end 35.14 30.97) (width 0.8) (layer "F.Cu") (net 9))
 (segment (start 33.99 36.26) (end 33.99 33.89) (width 0.8) (layer "F.Cu") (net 9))
 (segment (start 31.15 38.915) (end 31.15 37.4475) (width 0.3) (layer "F.Cu") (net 6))
 (segment (start 31.15 37.4475) (end 31.12 37.4175) (width 0.3) (layer "F.Cu") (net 6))
 (segment (start 68.12 40.22) (end 68.16 40.26) (width 0.3) (layer "F.Cu") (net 4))
 (segment (start 54.69 44.43) (end 54.04 45.08) (width 2) (layer "F.Cu") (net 4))
 (segment (start 71.925 40.595) (end 72.26 40.26) (width 0.3) (layer "F.Cu") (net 4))
 (segment (start 51.02 42.66) (end 52.65 44.29) (width 1) (layer "F.Cu") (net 4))
 (segment (start 45.35 42.54) (end 47.1 44.29) (width 1) (layer "F.Cu") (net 4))
 (segment (start 48.2 40.505) (end 50.775 40.505) (width 0.3) (layer "F.Cu") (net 4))
 (segment (start 39.69 40.26) (end 39.69 42.11) (width 1) (layer "F.Cu") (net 4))
 (segment (start 59.65 40.635) (end 60.575 40.635) (width 0.3) (layer "F.Cu") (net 4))
 (segment (start 54.04 45.08) (end 54.04 47.13) (width 2) (layer "F.Cu") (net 4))
 (segment (start 62.5 40.26) (end 62.5 42.78) (width 1) (layer "F.Cu") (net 4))
 (segment (start 50.775 40.505) (end 51.02 40.26) (width 0.3) (layer "F.Cu") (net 4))
 (segment (start 70.974 40.595) (end 71.925 40.595) (width 0.3) (layer "F.Cu") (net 4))
 (segment (start 51.02 40.26) (end 51.02 42.66) (width 1) (layer "F.Cu") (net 4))
 (segment (start 65.32 40.61) (end 66.63 40.61) (width 0.3) (layer "F.Cu") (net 4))
 (segment (start 54.69 44.43) (end 57.11 42.01) (width 1) (layer "F.Cu") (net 4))
 (segment (start 42.54 40.495) (end 45.115 40.495) (width 0.3) (layer "F.Cu") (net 4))
 (segment (start 72.26 40.26) (end 73.834 40.26) (width 0.3) (layer "F.Cu") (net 4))
 (segment (start 73.834 40.26) (end 73.834 43.076) (width 1) (layer "F.Cu") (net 4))
 (segment (start 45.115 40.495) (end 45.35 40.26) (width 0.3) (layer "F.Cu") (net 4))
 (segment (start 52.65 44.29) (end 47.1 44.29) (width 2) (layer "F.Cu") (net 4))
 (segment (start 68.16 40.26) (end 68.16 42.36) (width 1) (layer "F.Cu") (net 4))
 (segment (start 54.04 45.68) (end 52.71 44.35) (width 2) (layer "F.Cu") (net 4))
 (segment (start 73.834 43.076) (end 72.49 44.42) (width 1) (layer "F.Cu") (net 4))
 (segment (start 33.99 40.26) (end 33.99 42.42) (width 1) (layer "F.Cu") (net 4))
 (segment (start 41.87 44.29) (end 35.86 44.29) (width 2) (layer "F.Cu") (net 4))
 (segment (start 67.02 40.22) (end 68.12 40.22) (width 0.3) (layer "F.Cu") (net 4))
 (segment (start 55.51 40.26) (end 56.81 40.26) (width 0.3) (layer "F.Cu") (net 4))
 (segment (start 39.415 40.535) (end 39.69 40.26) (width 0.3) (layer "F.Cu") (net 4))
 (segment (start 56.81 40.26) (end 57.11 40.56) (width 0.3) (layer "F.Cu") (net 4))
 (segment (start 54.04 47.13) (end 54.04 45.68) (width 2) (layer "F.Cu") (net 4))
 (segment (start 52.71 44.35) (end 52.65 44.29) (width 2) (layer "F.Cu") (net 4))
 (segment (start 62.5 42.78) (end 60.86 44.42) (width 1) (layer "F.Cu") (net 4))
 (segment (start 54.7 44.42) (end 60.86 44.42) (width 2) (layer "F.Cu") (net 4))
 (segment (start 66.63 40.61) (end 67.02 40.22) (width 0.3) (layer "F.Cu") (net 4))
 (segment (start 45.35 40.26) (end 45.35 42.54) (width 1) (layer "F.Cu") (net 4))
 (segment (start 36.86 40.535) (end 39.415 40.535) (width 0.3) (layer "F.Cu") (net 4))
 (segment (start 60.575 40.635) (end 60.95 40.26) (width 0.3) (layer "F.Cu") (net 4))
 (segment (start 47.1 44.29) (end 41.87 44.29) (width 2) (layer "F.Cu") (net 4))
 (segment (start 60.86 44.42) (end 66.1 44.42) (width 2) (layer "F.Cu") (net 4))
 (segment (start 55.185 40.585) (end 55.51 40.26) (width 0.3) (layer "F.Cu") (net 4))
 (segment (start 66.1 44.42) (end 72.49 44.42) (width 2) (layer "F.Cu") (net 4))
 (segment (start 39.69 42.11) (end 41.87 44.29) (width 1) (layer "F.Cu") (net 4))
 (segment (start 33.685 40.565) (end 33.99 40.26) (width 0.3) (layer "F.Cu") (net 4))
 (segment (start 53.93 40.585) (end 55.185 40.585) (width 0.3) (layer "F.Cu") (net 4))
 (segment (start 31.15 40.565) (end 33.685 40.565) (width 0.3) (layer "F.Cu") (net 4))
 (segment (start 54.69 44.43) (end 54.7 44.42) (width 2) (layer "F.Cu") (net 4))
 (segment (start 57.11 42.01) (end 57.11 40.56) (width 1) (layer "F.Cu") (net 4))
 (segment (start 68.16 42.36) (end 66.1 44.42) (width 1) (layer "F.Cu") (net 4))
 (segment (start 33.99 42.42) (end 35.86 44.29) (width 1) (layer "F.Cu") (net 4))
 (segment (start 60.95 40.26) (end 62.5 40.26) (width 0.3) (layer "F.Cu") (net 4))
 (segment (start 62.48 36.24) (end 62.5 36.26) (width 0.8) (layer "F.Cu") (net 12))
 (segment (start 62.48 31.33) (end 62.48 36.24) (width 0.8) (layer "F.Cu") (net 12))
 (segment (start 62.12 30.97) (end 62.48 31.33) (width 0.8) (layer "F.Cu") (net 12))
 (segment (start 60.4325 35.5425) (end 61.15 36.26) (width 0.3) (layer "F.Cu") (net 12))
 (segment (start 59.64 35.5425) (end 60.4325 35.5425) (width 0.3) (layer "F.Cu") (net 12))
 (segment (start 61.15 36.26) (end 62.5 36.26) (width 0.3) (layer "F.Cu") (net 12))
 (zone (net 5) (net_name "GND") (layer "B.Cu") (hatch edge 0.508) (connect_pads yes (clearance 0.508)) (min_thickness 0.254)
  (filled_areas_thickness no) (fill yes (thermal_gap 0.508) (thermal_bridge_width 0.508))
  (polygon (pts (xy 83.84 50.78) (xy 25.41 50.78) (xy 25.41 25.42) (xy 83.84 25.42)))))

